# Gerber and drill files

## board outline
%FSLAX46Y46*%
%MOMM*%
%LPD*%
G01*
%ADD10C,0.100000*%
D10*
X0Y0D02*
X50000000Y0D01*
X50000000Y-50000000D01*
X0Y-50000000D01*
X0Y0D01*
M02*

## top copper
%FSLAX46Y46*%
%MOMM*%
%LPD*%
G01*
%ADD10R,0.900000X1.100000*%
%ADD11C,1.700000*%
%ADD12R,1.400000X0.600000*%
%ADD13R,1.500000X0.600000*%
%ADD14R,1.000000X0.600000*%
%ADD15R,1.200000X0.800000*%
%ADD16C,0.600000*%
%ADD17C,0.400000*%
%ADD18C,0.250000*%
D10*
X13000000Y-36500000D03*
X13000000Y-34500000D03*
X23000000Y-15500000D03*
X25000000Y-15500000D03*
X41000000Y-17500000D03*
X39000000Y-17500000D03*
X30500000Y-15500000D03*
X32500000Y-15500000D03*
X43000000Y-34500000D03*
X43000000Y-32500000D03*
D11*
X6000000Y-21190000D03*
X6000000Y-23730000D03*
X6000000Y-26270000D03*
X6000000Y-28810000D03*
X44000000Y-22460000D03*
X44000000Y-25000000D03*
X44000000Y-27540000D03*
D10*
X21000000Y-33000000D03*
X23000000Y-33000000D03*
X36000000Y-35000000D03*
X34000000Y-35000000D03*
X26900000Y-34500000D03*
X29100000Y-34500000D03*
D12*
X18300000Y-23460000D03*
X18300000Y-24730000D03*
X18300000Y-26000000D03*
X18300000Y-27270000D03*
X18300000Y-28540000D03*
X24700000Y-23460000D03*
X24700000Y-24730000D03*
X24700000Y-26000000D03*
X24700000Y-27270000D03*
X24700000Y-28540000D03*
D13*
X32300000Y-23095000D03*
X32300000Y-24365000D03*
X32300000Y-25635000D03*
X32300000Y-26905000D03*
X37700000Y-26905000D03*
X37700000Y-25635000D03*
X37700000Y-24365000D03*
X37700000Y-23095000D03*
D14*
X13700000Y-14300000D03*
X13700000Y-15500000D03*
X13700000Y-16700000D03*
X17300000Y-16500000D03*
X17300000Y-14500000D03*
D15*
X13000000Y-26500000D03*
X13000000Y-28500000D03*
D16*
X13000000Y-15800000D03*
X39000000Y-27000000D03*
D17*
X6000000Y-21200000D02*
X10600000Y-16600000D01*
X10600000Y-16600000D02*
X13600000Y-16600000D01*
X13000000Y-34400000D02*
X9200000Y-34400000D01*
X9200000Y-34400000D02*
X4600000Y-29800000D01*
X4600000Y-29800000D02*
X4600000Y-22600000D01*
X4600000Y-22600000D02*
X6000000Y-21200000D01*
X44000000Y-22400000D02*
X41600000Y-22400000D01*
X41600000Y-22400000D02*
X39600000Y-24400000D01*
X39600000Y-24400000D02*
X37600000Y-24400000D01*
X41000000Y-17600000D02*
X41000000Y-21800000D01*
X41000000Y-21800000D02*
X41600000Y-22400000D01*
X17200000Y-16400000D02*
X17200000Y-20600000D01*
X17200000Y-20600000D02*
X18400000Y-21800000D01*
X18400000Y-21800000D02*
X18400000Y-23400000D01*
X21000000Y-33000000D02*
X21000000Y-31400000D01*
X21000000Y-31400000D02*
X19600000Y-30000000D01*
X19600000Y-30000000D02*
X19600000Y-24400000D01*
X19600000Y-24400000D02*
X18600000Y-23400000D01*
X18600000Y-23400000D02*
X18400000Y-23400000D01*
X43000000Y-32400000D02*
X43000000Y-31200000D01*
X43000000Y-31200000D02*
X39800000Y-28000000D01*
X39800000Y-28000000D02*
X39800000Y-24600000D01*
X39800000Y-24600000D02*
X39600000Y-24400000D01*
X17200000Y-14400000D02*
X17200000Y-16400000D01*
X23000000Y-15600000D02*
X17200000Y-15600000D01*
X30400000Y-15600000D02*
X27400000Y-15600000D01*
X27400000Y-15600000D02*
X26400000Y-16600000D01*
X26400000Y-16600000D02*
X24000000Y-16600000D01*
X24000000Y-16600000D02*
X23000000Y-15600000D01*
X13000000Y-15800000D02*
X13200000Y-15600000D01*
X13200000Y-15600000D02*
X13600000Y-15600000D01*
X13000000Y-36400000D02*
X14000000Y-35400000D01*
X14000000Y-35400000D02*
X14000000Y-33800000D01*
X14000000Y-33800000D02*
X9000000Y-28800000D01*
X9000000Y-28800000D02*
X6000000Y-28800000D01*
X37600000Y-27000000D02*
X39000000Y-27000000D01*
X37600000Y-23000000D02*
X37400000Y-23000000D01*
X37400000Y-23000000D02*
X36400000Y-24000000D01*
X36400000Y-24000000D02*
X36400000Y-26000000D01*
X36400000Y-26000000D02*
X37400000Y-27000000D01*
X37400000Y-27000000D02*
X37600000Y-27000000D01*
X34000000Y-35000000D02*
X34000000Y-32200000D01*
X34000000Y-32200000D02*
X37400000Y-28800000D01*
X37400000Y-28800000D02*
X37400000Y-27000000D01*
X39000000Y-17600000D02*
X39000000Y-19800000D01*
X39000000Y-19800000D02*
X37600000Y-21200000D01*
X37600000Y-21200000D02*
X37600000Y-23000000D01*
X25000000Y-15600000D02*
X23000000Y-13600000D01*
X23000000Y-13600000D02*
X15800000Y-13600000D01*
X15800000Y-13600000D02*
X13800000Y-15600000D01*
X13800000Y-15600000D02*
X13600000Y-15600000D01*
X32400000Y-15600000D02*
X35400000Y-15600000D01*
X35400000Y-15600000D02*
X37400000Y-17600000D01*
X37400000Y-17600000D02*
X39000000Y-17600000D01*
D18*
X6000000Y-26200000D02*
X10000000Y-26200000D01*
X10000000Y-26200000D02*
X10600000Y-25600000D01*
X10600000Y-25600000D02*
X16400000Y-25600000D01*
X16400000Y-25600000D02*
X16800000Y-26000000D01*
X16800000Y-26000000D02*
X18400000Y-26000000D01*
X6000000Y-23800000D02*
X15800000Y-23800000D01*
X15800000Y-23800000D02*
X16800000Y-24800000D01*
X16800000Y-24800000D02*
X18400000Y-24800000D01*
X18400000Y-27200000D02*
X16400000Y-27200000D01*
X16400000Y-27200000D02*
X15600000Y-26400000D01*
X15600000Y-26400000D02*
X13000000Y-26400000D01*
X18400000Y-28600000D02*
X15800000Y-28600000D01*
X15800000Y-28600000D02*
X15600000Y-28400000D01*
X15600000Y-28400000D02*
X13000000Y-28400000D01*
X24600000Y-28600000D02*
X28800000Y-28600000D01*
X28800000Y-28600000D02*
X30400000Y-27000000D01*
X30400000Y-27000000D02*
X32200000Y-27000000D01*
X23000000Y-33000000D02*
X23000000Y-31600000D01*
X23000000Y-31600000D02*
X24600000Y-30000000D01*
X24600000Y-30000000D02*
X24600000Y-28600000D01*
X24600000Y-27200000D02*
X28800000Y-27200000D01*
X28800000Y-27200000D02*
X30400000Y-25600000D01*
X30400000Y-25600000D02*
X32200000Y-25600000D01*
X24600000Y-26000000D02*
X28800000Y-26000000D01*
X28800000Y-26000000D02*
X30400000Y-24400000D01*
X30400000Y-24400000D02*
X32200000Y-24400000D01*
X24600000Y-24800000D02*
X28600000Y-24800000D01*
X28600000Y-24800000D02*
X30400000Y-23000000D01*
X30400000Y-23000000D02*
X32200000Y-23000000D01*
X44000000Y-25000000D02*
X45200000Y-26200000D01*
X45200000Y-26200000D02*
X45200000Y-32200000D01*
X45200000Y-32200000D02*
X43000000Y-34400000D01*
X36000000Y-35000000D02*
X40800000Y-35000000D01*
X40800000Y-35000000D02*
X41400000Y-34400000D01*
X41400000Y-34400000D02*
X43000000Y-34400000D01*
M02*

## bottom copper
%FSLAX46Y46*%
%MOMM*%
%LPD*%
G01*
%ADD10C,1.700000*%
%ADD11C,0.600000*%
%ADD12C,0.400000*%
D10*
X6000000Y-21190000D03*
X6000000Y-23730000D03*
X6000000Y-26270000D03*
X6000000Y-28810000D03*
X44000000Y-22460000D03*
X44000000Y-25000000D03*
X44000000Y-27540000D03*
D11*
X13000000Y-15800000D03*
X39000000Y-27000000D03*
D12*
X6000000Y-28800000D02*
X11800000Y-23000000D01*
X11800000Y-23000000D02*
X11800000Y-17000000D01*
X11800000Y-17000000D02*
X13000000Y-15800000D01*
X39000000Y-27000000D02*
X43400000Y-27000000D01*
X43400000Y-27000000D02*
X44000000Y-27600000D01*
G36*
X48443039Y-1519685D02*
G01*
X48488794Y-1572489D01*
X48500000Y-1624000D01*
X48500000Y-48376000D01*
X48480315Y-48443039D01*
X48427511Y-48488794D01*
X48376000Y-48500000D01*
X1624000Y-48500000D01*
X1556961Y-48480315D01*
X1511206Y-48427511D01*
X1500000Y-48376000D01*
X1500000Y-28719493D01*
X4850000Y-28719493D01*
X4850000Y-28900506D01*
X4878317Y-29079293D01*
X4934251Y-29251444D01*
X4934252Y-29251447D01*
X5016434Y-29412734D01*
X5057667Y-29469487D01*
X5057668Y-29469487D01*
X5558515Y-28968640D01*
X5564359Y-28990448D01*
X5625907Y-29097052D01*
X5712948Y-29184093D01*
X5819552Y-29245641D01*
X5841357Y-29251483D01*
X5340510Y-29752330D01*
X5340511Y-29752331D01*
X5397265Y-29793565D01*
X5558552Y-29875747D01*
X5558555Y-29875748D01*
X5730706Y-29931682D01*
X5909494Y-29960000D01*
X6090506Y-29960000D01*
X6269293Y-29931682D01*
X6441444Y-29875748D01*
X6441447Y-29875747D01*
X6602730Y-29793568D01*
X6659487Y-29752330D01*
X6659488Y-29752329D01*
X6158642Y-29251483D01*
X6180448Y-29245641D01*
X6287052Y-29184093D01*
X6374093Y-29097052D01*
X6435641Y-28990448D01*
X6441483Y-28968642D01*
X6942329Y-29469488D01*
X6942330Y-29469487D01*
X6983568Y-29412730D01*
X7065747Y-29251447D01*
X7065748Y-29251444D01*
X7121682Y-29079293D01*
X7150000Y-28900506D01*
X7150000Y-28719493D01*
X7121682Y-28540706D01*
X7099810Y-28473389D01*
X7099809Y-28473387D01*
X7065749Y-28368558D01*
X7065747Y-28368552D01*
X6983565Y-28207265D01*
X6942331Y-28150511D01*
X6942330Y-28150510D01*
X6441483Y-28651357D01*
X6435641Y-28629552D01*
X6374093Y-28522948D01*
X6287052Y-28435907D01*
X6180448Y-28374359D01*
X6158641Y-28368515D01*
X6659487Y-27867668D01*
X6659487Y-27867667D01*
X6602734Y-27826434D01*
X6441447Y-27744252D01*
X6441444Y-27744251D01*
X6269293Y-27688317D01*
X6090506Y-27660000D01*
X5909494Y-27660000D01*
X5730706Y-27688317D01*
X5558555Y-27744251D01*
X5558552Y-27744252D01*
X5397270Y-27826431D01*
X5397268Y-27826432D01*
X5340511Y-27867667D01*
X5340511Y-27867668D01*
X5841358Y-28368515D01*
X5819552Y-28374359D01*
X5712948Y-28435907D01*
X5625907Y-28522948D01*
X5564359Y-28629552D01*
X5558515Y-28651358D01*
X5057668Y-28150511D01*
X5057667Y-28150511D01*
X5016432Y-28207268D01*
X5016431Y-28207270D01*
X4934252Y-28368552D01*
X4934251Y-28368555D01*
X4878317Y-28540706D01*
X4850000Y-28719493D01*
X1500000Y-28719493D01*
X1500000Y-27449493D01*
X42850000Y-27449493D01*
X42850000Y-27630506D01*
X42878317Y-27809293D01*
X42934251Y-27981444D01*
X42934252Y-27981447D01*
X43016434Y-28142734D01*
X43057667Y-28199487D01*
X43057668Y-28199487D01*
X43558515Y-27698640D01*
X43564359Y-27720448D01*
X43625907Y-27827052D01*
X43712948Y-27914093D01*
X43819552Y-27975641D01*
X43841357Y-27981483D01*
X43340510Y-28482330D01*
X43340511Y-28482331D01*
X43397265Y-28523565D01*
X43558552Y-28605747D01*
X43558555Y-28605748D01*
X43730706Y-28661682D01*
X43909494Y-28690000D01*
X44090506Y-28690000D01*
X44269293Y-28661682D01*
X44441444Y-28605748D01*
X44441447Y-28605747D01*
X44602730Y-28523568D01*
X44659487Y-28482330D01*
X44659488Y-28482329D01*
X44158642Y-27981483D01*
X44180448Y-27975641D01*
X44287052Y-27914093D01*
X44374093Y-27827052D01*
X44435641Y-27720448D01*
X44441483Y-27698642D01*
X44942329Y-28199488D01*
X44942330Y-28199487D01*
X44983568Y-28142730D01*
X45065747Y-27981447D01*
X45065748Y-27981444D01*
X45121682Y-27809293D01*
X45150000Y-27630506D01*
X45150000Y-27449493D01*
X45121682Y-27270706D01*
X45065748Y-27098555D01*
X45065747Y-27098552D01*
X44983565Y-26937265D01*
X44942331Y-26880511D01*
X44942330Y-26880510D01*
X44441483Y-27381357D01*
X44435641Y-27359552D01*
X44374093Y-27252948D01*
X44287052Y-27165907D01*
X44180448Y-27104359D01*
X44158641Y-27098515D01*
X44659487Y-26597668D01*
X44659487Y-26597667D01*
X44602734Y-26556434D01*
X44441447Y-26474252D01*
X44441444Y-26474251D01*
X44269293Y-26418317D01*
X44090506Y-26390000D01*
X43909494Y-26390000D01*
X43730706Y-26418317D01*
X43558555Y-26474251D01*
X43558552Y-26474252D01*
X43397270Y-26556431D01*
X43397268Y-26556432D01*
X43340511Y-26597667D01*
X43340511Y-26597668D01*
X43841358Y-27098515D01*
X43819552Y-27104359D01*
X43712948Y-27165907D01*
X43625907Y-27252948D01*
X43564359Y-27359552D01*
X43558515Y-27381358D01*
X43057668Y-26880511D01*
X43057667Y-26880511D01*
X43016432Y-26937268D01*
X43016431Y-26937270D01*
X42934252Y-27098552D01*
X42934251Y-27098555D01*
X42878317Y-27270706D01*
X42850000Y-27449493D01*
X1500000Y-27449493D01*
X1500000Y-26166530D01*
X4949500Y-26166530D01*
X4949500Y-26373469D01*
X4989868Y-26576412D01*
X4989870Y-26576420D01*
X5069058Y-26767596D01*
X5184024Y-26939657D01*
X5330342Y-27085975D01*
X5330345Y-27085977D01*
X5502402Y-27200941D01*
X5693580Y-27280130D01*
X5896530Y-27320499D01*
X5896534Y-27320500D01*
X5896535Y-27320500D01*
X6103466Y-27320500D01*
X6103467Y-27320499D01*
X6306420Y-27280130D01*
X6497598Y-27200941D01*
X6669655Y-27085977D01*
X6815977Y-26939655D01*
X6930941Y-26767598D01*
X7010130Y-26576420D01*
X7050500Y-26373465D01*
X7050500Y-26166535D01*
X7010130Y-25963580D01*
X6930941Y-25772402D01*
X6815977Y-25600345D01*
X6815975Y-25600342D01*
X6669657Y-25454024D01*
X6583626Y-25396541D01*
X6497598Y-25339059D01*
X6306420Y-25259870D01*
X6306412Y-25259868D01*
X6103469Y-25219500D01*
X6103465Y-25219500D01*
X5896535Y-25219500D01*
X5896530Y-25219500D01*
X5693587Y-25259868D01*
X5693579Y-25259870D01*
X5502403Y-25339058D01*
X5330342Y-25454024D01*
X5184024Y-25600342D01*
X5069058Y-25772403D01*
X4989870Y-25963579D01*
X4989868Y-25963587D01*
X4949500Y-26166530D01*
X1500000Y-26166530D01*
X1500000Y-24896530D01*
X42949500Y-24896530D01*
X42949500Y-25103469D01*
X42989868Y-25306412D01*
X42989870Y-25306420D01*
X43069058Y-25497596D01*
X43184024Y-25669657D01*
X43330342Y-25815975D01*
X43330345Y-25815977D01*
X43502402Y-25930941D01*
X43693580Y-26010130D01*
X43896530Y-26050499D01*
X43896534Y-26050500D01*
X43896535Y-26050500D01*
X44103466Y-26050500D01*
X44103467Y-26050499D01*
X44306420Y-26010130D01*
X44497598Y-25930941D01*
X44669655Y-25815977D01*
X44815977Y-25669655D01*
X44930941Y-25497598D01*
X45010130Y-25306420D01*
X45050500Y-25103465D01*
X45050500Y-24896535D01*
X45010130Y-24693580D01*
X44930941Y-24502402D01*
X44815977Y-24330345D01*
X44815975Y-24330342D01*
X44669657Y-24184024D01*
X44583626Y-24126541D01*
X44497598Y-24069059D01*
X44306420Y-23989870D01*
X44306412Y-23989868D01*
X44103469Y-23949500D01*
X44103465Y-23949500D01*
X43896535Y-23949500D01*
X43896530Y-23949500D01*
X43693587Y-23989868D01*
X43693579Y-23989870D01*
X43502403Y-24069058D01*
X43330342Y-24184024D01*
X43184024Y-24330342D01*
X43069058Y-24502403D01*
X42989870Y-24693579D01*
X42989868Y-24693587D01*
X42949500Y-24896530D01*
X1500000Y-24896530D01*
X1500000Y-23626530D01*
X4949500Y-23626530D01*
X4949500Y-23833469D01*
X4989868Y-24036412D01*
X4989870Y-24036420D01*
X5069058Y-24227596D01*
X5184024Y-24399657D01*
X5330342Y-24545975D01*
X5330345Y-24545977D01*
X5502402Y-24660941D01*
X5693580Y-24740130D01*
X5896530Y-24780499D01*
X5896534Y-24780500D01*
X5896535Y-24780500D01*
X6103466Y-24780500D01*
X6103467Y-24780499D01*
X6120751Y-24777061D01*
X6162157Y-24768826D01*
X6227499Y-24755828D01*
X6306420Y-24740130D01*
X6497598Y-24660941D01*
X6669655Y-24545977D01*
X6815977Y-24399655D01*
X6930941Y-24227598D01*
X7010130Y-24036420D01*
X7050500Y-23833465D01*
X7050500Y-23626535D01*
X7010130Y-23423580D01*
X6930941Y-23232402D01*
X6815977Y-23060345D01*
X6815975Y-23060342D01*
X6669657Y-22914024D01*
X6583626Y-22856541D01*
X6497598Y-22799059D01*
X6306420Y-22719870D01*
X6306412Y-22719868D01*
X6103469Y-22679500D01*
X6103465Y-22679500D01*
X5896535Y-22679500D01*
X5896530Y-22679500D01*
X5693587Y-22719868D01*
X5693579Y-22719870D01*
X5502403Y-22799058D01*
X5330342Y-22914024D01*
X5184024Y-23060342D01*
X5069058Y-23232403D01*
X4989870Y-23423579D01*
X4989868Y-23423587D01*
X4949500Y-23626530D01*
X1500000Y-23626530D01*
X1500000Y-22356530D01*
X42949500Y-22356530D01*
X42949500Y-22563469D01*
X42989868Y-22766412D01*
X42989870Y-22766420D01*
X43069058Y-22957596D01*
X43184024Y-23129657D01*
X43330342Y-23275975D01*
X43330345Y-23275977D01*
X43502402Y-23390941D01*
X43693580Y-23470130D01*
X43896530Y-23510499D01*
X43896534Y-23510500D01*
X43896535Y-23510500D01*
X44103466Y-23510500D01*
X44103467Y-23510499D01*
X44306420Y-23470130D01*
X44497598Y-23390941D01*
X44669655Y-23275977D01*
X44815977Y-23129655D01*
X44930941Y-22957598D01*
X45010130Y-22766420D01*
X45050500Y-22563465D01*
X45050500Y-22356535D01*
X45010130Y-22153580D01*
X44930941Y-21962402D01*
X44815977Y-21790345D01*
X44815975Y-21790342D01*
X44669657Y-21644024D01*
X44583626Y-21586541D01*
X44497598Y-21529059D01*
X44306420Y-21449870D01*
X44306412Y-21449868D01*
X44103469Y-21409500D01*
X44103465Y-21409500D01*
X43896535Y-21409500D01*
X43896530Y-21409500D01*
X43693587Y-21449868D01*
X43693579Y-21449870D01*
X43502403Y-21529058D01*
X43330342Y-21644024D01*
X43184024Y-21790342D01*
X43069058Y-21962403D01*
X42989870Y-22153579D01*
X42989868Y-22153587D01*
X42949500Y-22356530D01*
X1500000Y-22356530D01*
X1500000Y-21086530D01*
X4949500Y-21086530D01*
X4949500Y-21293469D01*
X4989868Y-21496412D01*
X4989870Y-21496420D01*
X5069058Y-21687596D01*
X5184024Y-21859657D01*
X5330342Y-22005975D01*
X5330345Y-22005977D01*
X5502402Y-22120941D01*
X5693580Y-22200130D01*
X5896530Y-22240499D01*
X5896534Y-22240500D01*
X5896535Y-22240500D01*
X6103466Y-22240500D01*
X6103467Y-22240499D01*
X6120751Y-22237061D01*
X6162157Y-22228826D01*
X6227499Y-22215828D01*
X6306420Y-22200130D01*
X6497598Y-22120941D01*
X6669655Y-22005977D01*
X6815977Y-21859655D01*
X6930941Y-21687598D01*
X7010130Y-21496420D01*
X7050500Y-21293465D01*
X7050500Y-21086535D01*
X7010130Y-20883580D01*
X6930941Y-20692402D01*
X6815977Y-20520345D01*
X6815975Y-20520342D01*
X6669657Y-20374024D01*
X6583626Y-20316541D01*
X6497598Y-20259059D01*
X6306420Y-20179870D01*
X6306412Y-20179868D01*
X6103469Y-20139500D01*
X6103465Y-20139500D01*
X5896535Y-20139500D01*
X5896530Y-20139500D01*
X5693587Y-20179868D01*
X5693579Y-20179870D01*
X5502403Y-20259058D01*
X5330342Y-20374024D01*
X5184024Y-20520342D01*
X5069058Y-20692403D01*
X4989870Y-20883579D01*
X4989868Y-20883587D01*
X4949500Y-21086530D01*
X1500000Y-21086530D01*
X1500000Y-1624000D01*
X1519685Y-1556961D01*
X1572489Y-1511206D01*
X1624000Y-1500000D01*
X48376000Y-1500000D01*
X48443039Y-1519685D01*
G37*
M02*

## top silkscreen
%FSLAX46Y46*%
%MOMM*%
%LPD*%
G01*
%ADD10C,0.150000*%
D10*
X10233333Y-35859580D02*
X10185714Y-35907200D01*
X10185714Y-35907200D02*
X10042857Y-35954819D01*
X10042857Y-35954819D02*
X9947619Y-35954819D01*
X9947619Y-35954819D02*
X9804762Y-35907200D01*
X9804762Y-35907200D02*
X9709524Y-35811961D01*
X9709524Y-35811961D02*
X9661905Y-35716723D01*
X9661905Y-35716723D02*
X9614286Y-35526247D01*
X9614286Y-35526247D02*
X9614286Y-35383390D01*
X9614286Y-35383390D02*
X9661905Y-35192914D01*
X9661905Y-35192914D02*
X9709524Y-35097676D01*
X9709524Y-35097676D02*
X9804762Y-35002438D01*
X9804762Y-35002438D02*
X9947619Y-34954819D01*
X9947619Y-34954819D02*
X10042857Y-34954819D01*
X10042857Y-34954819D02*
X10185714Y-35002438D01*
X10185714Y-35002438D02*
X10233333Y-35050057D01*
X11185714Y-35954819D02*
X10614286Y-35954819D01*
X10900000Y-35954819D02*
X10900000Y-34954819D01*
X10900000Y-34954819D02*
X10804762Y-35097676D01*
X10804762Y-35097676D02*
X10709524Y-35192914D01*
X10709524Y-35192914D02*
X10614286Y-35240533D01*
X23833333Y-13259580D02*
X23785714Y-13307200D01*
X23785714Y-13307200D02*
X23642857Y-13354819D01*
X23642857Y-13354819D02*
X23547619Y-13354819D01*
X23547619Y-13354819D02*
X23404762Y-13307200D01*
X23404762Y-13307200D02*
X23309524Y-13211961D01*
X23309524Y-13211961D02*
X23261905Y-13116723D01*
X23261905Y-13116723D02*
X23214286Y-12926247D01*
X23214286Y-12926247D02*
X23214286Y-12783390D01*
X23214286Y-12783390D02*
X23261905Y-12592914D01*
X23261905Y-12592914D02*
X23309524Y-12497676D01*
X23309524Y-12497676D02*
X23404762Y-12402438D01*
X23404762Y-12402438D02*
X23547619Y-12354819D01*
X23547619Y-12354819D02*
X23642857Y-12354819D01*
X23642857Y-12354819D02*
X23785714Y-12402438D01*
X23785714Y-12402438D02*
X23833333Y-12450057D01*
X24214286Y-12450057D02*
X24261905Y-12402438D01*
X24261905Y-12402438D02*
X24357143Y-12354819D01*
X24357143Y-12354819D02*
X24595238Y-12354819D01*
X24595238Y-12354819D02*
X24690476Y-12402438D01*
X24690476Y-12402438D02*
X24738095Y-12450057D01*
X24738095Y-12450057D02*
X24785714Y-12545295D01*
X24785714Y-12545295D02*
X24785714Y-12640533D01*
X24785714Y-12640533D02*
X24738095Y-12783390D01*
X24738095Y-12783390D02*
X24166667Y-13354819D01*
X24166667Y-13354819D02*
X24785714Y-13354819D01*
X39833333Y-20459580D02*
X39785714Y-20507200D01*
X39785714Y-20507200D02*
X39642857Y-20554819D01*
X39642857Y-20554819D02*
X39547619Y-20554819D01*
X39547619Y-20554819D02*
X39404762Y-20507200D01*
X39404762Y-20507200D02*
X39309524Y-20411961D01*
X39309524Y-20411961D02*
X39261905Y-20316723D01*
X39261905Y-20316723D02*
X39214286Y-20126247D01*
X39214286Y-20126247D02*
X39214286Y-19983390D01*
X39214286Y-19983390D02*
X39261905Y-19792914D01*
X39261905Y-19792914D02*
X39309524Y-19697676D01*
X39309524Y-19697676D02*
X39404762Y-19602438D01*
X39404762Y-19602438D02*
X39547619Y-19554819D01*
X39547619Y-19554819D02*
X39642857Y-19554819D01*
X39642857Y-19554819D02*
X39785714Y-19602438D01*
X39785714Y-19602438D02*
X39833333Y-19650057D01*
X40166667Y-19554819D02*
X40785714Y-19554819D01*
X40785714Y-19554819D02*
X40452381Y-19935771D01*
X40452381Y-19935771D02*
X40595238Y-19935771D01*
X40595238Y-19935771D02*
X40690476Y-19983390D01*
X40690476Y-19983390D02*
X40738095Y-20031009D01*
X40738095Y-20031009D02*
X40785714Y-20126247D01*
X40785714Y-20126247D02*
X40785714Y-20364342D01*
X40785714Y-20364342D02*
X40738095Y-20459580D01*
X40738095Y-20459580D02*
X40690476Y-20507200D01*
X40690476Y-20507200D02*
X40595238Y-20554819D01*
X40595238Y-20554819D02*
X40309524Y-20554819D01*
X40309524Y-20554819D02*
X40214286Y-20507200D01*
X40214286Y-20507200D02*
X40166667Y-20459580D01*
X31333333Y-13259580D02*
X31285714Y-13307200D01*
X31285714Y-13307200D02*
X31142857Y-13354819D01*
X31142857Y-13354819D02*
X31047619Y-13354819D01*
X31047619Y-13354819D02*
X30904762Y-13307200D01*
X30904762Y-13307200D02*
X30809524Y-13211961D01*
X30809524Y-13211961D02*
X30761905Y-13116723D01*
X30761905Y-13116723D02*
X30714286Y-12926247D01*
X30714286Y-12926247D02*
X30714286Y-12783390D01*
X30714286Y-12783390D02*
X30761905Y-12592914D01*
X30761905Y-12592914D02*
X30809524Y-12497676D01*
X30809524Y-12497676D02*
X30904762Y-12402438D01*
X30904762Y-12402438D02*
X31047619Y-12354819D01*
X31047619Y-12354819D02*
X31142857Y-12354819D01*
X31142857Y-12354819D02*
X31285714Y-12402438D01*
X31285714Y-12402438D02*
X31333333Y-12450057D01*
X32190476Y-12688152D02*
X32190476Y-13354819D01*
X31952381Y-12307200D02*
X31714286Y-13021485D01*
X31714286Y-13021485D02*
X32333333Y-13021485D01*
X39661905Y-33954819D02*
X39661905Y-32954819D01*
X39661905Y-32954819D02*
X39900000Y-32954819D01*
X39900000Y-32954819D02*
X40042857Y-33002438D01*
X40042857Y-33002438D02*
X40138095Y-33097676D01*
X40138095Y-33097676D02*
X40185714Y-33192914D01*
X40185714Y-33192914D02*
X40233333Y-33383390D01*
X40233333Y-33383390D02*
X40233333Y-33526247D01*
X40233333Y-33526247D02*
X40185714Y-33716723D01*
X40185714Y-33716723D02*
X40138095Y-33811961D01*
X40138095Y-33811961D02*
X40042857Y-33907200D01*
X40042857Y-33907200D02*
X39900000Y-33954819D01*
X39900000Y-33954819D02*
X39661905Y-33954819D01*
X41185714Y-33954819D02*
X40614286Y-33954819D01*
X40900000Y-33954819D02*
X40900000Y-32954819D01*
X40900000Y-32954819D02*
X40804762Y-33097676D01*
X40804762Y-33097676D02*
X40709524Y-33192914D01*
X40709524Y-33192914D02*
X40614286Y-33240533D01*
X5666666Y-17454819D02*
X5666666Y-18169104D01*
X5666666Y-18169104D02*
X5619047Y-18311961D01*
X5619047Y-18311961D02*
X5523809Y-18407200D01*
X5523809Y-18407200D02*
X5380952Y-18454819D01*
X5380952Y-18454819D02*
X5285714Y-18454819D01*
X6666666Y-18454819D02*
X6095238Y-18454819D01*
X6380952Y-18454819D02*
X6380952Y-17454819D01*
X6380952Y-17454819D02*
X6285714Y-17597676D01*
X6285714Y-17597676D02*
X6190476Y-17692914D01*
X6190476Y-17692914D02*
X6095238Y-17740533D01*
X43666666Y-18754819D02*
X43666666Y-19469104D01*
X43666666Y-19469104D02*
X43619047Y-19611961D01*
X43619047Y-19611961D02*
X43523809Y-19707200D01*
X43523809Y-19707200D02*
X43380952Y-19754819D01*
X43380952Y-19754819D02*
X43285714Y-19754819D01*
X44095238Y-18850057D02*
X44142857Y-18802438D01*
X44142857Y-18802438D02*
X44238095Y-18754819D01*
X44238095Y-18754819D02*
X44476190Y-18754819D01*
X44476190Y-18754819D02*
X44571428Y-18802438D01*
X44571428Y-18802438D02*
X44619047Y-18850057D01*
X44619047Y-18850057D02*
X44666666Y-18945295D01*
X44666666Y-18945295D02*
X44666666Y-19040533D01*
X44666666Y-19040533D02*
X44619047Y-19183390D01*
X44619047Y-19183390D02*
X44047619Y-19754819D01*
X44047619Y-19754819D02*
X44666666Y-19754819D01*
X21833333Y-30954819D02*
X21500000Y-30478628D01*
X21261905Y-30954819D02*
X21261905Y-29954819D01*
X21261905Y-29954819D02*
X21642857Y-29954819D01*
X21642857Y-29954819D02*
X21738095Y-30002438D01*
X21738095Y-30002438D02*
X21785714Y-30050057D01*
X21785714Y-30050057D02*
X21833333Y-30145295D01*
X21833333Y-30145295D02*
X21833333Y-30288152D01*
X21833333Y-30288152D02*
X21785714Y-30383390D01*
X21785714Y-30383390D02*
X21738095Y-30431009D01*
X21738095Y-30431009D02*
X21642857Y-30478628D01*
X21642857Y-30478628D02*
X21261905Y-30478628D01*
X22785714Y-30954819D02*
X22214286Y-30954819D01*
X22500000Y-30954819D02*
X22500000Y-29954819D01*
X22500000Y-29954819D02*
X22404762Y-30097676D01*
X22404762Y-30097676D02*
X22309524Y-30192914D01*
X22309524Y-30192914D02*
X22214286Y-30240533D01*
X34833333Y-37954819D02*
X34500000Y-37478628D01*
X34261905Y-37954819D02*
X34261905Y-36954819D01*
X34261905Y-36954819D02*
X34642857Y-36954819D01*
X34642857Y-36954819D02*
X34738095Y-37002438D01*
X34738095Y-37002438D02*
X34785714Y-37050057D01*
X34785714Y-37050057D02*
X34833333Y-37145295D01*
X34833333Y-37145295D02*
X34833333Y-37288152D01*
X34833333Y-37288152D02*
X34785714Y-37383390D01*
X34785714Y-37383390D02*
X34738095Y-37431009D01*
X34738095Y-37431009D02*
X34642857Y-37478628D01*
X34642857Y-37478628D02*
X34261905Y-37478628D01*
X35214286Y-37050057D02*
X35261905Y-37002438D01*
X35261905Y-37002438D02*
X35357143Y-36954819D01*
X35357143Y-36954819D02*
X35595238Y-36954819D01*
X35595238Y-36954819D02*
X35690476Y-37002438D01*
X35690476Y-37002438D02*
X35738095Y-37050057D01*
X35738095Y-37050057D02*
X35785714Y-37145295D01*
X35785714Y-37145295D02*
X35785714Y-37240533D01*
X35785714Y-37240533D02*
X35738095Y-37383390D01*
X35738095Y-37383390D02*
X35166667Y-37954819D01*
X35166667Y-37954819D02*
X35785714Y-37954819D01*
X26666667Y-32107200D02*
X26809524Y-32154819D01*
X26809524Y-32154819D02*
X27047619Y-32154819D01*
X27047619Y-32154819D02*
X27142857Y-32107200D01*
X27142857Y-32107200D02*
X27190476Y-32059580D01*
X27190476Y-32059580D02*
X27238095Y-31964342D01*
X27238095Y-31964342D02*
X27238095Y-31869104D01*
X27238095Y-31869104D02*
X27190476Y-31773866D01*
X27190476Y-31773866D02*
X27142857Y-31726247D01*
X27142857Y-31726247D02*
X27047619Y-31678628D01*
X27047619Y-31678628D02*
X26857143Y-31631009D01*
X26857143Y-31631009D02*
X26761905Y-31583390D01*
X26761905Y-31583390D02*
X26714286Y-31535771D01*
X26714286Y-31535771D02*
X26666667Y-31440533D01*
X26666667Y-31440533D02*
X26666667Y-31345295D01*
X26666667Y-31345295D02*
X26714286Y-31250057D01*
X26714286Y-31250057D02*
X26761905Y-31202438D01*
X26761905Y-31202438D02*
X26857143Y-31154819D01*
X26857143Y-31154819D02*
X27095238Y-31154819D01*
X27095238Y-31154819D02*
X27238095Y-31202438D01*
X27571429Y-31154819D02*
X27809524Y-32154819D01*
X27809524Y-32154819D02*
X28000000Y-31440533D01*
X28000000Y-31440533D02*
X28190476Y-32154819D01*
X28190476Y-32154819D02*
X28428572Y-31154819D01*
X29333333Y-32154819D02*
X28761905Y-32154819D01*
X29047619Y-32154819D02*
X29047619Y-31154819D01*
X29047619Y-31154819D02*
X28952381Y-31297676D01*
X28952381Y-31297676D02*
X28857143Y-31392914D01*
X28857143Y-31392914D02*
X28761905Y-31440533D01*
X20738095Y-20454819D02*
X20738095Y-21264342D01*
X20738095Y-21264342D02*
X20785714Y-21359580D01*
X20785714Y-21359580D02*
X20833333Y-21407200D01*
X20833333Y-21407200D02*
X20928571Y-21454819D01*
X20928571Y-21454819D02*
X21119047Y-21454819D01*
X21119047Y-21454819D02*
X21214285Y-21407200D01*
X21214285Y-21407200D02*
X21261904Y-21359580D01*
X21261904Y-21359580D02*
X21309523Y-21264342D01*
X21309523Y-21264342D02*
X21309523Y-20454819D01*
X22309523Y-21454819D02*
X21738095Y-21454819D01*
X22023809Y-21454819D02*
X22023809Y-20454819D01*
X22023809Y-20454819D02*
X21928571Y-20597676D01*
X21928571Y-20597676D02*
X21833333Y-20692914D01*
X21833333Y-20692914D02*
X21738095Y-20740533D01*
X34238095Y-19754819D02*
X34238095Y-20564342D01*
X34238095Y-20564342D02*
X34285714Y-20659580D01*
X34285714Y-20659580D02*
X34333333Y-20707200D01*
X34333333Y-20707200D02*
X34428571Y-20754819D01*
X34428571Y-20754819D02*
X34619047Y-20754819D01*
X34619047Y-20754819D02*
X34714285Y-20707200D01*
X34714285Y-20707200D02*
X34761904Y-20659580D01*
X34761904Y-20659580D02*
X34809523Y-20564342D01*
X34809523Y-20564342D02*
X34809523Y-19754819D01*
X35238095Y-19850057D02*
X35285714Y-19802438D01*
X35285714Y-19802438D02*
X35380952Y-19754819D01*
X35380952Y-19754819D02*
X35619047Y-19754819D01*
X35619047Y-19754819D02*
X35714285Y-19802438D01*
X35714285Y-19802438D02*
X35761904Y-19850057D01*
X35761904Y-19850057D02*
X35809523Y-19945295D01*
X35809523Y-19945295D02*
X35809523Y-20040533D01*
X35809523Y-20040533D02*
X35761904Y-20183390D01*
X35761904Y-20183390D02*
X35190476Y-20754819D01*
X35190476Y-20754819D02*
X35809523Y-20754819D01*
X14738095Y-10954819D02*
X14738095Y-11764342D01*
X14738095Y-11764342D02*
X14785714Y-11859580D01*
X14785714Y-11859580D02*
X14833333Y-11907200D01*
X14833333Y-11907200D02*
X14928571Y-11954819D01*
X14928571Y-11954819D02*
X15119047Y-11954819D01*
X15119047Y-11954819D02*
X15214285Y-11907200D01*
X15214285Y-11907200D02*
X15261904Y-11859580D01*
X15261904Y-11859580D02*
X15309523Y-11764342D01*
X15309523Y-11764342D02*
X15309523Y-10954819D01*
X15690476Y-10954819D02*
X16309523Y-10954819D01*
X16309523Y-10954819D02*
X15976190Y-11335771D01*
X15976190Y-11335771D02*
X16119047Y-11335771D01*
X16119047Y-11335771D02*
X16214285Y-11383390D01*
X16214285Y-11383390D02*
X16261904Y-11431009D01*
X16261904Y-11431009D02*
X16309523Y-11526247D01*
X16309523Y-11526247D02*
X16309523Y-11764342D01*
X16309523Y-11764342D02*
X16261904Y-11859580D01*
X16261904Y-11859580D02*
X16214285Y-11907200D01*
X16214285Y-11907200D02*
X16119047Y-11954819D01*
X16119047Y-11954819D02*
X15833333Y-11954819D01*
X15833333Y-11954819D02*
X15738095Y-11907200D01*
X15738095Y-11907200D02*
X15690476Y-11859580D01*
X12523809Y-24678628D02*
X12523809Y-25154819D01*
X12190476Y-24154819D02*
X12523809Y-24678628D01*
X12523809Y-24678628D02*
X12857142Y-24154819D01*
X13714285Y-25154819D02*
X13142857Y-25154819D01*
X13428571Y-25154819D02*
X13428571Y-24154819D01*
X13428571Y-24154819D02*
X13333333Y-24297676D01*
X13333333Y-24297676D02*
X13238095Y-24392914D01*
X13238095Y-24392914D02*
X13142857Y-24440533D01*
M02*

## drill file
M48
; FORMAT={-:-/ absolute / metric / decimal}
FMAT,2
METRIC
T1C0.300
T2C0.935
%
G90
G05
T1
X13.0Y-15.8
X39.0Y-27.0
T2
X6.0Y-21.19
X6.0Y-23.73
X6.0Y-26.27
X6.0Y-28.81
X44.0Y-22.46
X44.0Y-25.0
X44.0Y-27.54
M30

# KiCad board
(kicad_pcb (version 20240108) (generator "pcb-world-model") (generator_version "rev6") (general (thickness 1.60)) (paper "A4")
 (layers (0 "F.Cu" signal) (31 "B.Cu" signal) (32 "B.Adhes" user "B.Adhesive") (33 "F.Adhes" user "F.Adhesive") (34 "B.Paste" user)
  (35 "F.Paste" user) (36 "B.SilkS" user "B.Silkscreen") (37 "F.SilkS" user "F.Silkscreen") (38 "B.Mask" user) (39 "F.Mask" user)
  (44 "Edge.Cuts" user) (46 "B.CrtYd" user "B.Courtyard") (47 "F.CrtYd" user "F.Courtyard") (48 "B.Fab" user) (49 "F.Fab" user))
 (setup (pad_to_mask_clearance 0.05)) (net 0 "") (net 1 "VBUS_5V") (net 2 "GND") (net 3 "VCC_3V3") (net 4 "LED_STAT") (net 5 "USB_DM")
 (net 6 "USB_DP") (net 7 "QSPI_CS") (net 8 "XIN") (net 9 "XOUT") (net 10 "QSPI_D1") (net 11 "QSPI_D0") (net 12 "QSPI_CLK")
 (gr_rect (start 0.0 0.0) (end 50.0000 50.0000) (stroke (width 0.1) (type default)) (fill none) (layer "Edge.Cuts"))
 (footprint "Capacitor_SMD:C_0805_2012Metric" (layer "F.Cu") (at 13.0000 35.5000 90)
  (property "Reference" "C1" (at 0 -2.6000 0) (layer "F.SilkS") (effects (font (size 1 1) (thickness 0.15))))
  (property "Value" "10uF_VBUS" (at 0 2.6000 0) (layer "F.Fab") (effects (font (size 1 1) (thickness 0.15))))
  (pad "1" smd rect (at -1.0000 0.0000) (size 0.9000 1.1000) (layers "F.Cu" "F.Paste" "F.Mask") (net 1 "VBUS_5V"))
  (pad "2" smd rect (at 1.0000 0.0000) (size 0.9000 1.1000) (layers "F.Cu" "F.Paste" "F.Mask") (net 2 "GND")))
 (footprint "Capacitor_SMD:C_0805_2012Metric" (layer "F.Cu") (at 24.0000 15.5000 0)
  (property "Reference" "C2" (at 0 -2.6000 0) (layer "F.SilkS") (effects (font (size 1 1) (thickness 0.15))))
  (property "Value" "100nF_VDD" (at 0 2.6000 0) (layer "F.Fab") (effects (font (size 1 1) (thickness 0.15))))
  (pad "1" smd rect (at -1.0000 0.0000) (size 0.9000 1.1000) (layers "F.Cu" "F.Paste" "F.Mask") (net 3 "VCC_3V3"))
  (pad "2" smd rect (at 1.0000 0.0000) (size 0.9000 1.1000) (layers "F.Cu" "F.Paste" "F.Mask") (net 2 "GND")))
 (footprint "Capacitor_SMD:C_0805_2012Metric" (layer "F.Cu") (at 40.0000 17.5000 180)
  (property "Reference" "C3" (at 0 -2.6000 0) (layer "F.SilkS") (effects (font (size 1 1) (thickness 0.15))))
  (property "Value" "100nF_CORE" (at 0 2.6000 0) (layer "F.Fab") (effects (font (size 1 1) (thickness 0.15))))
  (pad "1" smd rect (at -1.0000 0.0000) (size 0.9000 1.1000) (layers "F.Cu" "F.Paste" "F.Mask") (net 3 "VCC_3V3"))
  (pad "2" smd rect (at 1.0000 0.0000) (size 0.9000 1.1000) (layers "F.Cu" "F.Paste" "F.Mask") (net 2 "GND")))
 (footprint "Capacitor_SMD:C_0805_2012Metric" (layer "F.Cu") (at 31.5000 15.5000 0)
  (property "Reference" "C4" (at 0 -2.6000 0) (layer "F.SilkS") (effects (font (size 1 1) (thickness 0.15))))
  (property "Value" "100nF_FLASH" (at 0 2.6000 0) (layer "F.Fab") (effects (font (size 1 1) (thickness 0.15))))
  (pad "1" smd rect (at -1.0000 0.0000) (size 0.9000 1.1000) (layers "F.Cu" "F.Paste" "F.Mask") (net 3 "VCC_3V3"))
  (pad "2" smd rect (at 1.0000 0.0000) (size 0.9000 1.1000) (layers "F.Cu" "F.Paste" "F.Mask") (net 2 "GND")))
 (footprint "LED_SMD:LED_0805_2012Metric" (layer "F.Cu") (at 43.0000 33.5000 90)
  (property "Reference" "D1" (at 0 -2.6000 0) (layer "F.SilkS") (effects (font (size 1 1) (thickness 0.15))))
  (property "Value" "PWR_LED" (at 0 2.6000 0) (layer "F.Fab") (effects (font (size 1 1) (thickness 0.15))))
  (pad "1" smd rect (at -1.0000 0.0000) (size 0.9000 1.1000) (layers "F.Cu" "F.Paste" "F.Mask") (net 3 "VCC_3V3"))
  (pad "2" smd rect (at 1.0000 0.0000) (size 0.9000 1.1000) (layers "F.Cu" "F.Paste" "F.Mask") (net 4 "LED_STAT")))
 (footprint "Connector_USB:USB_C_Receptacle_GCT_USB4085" (layer "F.Cu") (at 6.0000 25.0000 0) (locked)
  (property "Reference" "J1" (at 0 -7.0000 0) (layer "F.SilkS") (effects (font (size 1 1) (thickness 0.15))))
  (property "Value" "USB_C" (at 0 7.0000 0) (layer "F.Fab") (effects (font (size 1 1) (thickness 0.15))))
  (pad "1" thru_hole circle (at 0.0000 -3.8100) (size 1.7000 1.7000) (drill 0.9350) (layers "*.Cu" "*.Mask") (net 1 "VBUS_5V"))
  (pad "2" thru_hole circle (at 0.0000 -1.2700) (size 1.7000 1.7000) (drill 0.9350) (layers "*.Cu" "*.Mask") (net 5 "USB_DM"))
  (pad "3" thru_hole circle (at 0.0000 1.2700) (size 1.7000 1.7000) (drill 0.9350) (layers "*.Cu" "*.Mask") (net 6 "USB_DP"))
  (pad "4" thru_hole circle (at 0.0000 3.8100) (size 1.7000 1.7000) (drill 0.9350) (layers "*.Cu" "*.Mask") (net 2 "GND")))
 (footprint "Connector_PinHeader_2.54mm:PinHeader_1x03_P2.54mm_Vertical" (layer "F.Cu") (at 44.0000 25.0000 0) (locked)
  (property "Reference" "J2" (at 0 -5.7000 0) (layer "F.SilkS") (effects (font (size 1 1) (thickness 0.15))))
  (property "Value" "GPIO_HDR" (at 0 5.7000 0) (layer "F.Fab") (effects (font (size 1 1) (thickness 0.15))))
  (pad "1" thru_hole circle (at 0.0000 -2.5400) (size 1.7000 1.7000) (drill 0.9350) (layers "*.Cu" "*.Mask") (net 3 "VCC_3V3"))
  (pad "2" thru_hole circle (at 0.0000 0.0000) (size 1.7000 1.7000) (drill 0.9350) (layers "*.Cu" "*.Mask") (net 4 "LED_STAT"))
  (pad "3" thru_hole circle (at 0.0000 2.5400) (size 1.7000 1.7000) (drill 0.9350) (layers "*.Cu" "*.Mask") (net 2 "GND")))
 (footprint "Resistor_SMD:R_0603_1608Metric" (layer "F.Cu") (at 22.0000 33.0000 0)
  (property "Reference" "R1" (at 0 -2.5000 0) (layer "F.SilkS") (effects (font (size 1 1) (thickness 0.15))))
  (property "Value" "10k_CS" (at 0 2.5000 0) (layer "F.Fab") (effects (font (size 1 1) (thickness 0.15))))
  (pad "1" smd rect (at -1.0000 0.0000) (size 0.9000 1.1000) (layers "F.Cu" "F.Paste" "F.Mask") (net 3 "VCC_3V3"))
  (pad "2" smd rect (at 1.0000 0.0000) (size 0.9000 1.1000) (layers "F.Cu" "F.Paste" "F.Mask") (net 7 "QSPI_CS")))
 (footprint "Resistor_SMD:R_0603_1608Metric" (layer "F.Cu") (at 35.0000 35.0000 180)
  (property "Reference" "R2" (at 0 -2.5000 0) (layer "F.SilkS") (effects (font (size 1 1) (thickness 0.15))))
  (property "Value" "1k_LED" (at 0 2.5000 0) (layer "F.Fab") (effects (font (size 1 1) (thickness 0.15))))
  (pad "1" smd rect (at -1.0000 0.0000) (size 0.9000 1.1000) (layers "F.Cu" "F.Paste" "F.Mask") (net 4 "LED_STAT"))
  (pad "2" smd rect (at 1.0000 0.0000) (size 0.9000 1.1000) (layers "F.Cu" "F.Paste" "F.Mask") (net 2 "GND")))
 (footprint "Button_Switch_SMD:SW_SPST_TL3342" (layer "F.Cu") (at 28.0000 34.5000 0)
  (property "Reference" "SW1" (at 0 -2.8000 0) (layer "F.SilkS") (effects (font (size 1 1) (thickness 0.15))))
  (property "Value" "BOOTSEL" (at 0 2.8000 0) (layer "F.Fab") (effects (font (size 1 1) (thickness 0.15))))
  (pad "1" smd rect (at -1.1000 0.0000) (size 0.9000 1.1000) (layers "F.Cu" "F.Paste" "F.Mask") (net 7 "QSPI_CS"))
  (pad "2" smd rect (at 1.1000 0.0000) (size 0.9000 1.1000) (layers "F.Cu" "F.Paste" "F.Mask") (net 2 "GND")))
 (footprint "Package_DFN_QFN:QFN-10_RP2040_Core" (layer "F.Cu") (at 21.5000 26.0000 0)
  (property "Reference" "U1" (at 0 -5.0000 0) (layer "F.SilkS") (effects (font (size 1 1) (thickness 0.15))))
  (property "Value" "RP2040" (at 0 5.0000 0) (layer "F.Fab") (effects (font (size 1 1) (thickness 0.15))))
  (pad "1" smd rect (at -3.2000 -2.5400) (size 1.4000 0.6000) (layers "F.Cu" "F.Paste" "F.Mask") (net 3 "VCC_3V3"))
  (pad "2" smd rect (at -3.2000 -1.2700) (size 1.4000 0.6000) (layers "F.Cu" "F.Paste" "F.Mask") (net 5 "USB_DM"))
  (pad "3" smd rect (at -3.2000 0.0000) (size 1.4000 0.6000) (layers "F.Cu" "F.Paste" "F.Mask") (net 6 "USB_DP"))
  (pad "4" smd rect (at -3.2000 1.2700) (size 1.4000 0.6000) (layers "F.Cu" "F.Paste" "F.Mask") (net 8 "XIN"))
  (pad "5" smd rect (at -3.2000 2.5400) (size 1.4000 0.6000) (layers "F.Cu" "F.Paste" "F.Mask") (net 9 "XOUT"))
  (pad "6" smd rect (at 3.2000 -2.5400) (size 1.4000 0.6000) (layers "F.Cu" "F.Paste" "F.Mask") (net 4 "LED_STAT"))
  (pad "7" smd rect (at 3.2000 -1.2700) (size 1.4000 0.6000) (layers "F.Cu" "F.Paste" "F.Mask") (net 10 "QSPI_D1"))
  (pad "8" smd rect (at 3.2000 0.0000) (size 1.4000 0.6000) (layers "F.Cu" "F.Paste" "F.Mask") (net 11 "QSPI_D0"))
  (pad "9" smd rect (at 3.2000 1.2700) (size 1.4000 0.6000) (layers "F.Cu" "F.Paste" "F.Mask") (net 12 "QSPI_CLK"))
  (pad "10" smd rect (at 3.2000 2.5400) (size 1.4000 0.6000) (layers "F.Cu" "F.Paste" "F.Mask") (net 7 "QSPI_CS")))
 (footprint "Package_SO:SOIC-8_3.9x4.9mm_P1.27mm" (layer "F.Cu") (at 35.0000 25.0000 0)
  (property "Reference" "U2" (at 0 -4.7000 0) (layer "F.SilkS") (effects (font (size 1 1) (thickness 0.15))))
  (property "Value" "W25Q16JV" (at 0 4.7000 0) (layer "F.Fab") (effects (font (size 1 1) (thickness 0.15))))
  (pad "1" smd rect (at -2.7000 -1.9050) (size 1.5000 0.6000) (layers "F.Cu" "F.Paste" "F.Mask") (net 10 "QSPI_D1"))
  (pad "2" smd rect (at -2.7000 -0.6350) (size 1.5000 0.6000) (layers "F.Cu" "F.Paste" "F.Mask") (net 11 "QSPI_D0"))
  (pad "3" smd rect (at -2.7000 0.6350) (size 1.5000 0.6000) (layers "F.Cu" "F.Paste" "F.Mask") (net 12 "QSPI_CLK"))
  (pad "4" smd rect (at -2.7000 1.9050) (size 1.5000 0.6000) (layers "F.Cu" "F.Paste" "F.Mask") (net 7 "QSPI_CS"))
  (pad "5" smd rect (at 2.7000 1.9050) (size 1.5000 0.6000) (layers "F.Cu" "F.Paste" "F.Mask") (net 2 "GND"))
  (pad "6" smd rect (at 2.7000 0.6350) (size 1.5000 0.6000) (layers "F.Cu" "F.Paste" "F.Mask") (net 3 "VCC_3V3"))
  (pad "7" smd rect (at 2.7000 -0.6350) (size 1.5000 0.6000) (layers "F.Cu" "F.Paste" "F.Mask") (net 3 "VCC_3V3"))
  (pad "8" smd rect (at 2.7000 -1.9050) (size 1.5000 0.6000) (layers "F.Cu" "F.Paste" "F.Mask") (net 2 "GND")))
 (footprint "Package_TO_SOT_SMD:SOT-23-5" (layer "F.Cu") (at 15.5000 15.5000 0)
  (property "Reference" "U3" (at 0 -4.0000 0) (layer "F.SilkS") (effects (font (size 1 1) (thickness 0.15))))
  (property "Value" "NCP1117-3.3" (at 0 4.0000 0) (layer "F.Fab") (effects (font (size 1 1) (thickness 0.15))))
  (pad "1" smd rect (at -1.8000 -1.2000) (size 1.0000 0.6000) (layers "F.Cu" "F.Paste" "F.Mask") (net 1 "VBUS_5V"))
  (pad "2" smd rect (at -1.8000 0.0000) (size 1.0000 0.6000) (layers "F.Cu" "F.Paste" "F.Mask") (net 2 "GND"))
  (pad "3" smd rect (at -1.8000 1.2000) (size 1.0000 0.6000) (layers "F.Cu" "F.Paste" "F.Mask") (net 1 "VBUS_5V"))
  (pad "4" smd rect (at 1.8000 1.0000) (size 1.0000 0.6000) (layers "F.Cu" "F.Paste" "F.Mask") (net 3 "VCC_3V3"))
  (pad "5" smd rect (at 1.8000 -1.0000) (size 1.0000 0.6000) (layers "F.Cu" "F.Paste" "F.Mask") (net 3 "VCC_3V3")))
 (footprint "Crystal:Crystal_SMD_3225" (layer "F.Cu") (at 13.0000 27.5000 0)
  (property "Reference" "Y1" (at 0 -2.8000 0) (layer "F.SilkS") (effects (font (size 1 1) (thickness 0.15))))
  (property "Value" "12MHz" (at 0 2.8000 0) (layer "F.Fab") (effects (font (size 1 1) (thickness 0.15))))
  (pad "1" smd rect (at 0.0000 -1.0000) (size 1.2000 0.8000) (layers "F.Cu" "F.Paste" "F.Mask") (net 8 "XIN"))
  (pad "2" smd rect (at 0.0000 1.0000) (size 1.2000 0.8000) (layers "F.Cu" "F.Paste" "F.Mask") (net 9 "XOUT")))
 (segment (start 6.0000 21.2000) (end 10.6000 16.6000) (width 0.4000) (layer "F.Cu") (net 1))
 (segment (start 10.6000 16.6000) (end 13.6000 16.6000) (width 0.4000) (layer "F.Cu") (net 1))
 (segment (start 13.0000 34.4000) (end 9.2000 34.4000) (width 0.4000) (layer "F.Cu") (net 1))
 (segment (start 9.2000 34.4000) (end 4.6000 29.8000) (width 0.4000) (layer "F.Cu") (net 1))
 (segment (start 4.6000 29.8000) (end 4.6000 22.6000) (width 0.4000) (layer "F.Cu") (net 1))
 (segment (start 4.6000 22.6000) (end 6.0000 21.2000) (width 0.4000) (layer "F.Cu") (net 1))
 (segment (start 44.0000 22.4000) (end 41.6000 22.4000) (width 0.4000) (layer "F.Cu") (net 3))
 (segment (start 41.6000 22.4000) (end 39.6000 24.4000) (width 0.4000) (layer "F.Cu") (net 3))
 (segment (start 39.6000 24.4000) (end 37.6000 24.4000) (width 0.4000) (layer "F.Cu") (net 3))
 (segment (start 41.0000 17.6000) (end 41.0000 21.8000) (width 0.4000) (layer "F.Cu") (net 3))
 (segment (start 41.0000 21.8000) (end 41.6000 22.4000) (width 0.4000) (layer "F.Cu") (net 3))
 (segment (start 17.2000 16.4000) (end 17.2000 20.6000) (width 0.4000) (layer "F.Cu") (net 3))
 (segment (start 17.2000 20.6000) (end 18.4000 21.8000) (width 0.4000) (layer "F.Cu") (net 3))
 (segment (start 18.4000 21.8000) (end 18.4000 23.4000) (width 0.4000) (layer "F.Cu") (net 3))
 (segment (start 21.0000 33.0000) (end 21.0000 31.4000) (width 0.4000) (layer "F.Cu") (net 3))
 (segment (start 21.0000 31.4000) (end 19.6000 30.0000) (width 0.4000) (layer "F.Cu") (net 3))
 (segment (start 19.6000 30.0000) (end 19.6000 24.4000) (width 0.4000) (layer "F.Cu") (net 3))
 (segment (start 19.6000 24.4000) (end 18.6000 23.4000) (width 0.4000) (layer "F.Cu") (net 3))
 (segment (start 18.6000 23.4000) (end 18.4000 23.4000) (width 0.4000) (layer "F.Cu") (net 3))
 (segment (start 43.0000 32.4000) (end 43.0000 31.2000) (width 0.4000) (layer "F.Cu") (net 3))
 (segment (start 43.0000 31.2000) (end 39.8000 28.0000) (width 0.4000) (layer "F.Cu") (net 3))
 (segment (start 39.8000 28.0000) (end 39.8000 24.6000) (width 0.4000) (layer "F.Cu") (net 3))
 (segment (start 39.8000 24.6000) (end 39.6000 24.4000) (width 0.4000) (layer "F.Cu") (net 3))
 (segment (start 17.2000 14.4000) (end 17.2000 16.4000) (width 0.4000) (layer "F.Cu") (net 3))
 (segment (start 23.0000 15.6000) (end 17.2000 15.6000) (width 0.4000) (layer "F.Cu") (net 3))
 (segment (start 30.4000 15.6000) (end 27.4000 15.6000) (width 0.4000) (layer "F.Cu") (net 3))
 (segment (start 27.4000 15.6000) (end 26.4000 16.6000) (width 0.4000) (layer "F.Cu") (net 3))
 (segment (start 26.4000 16.6000) (end 24.0000 16.6000) (width 0.4000) (layer "F.Cu") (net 3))
 (segment (start 24.0000 16.6000) (end 23.0000 15.6000) (width 0.4000) (layer "F.Cu") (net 3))
 (segment (start 6.0000 28.8000) (end 11.8000 23.0000) (width 0.4000) (layer "B.Cu") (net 2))
 (segment (start 11.8000 23.0000) (end 11.8000 17.0000) (width 0.4000) (layer "B.Cu") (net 2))
 (segment (start 11.8000 17.0000) (end 13.0000 15.8000) (width 0.4000) (layer "B.Cu") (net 2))
 (segment (start 13.0000 15.8000) (end 13.2000 15.6000) (width 0.4000) (layer "F.Cu") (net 2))
 (segment (start 13.2000 15.6000) (end 13.6000 15.6000) (width 0.4000) (layer "F.Cu") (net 2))
 (segment (start 13.0000 36.4000) (end 14.0000 35.4000) (width 0.4000) (layer "F.Cu") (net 2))
 (segment (start 14.0000 35.4000) (end 14.0000 33.8000) (width 0.4000) (layer "F.Cu") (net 2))
 (segment (start 14.0000 33.8000) (end 9.0000 28.8000) (width 0.4000) (layer "F.Cu") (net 2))
 (segment (start 9.0000 28.8000) (end 6.0000 28.8000) (width 0.4000) (layer "F.Cu") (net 2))
 (segment (start 37.6000 27.0000) (end 39.0000 27.0000) (width 0.4000) (layer "F.Cu") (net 2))
 (segment (start 39.0000 27.0000) (end 43.4000 27.0000) (width 0.4000) (layer "B.Cu") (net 2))
 (segment (start 43.4000 27.0000) (end 44.0000 27.6000) (width 0.4000) (layer "B.Cu") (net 2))
 (segment (start 37.6000 23.0000) (end 37.4000 23.0000) (width 0.4000) (layer "F.Cu") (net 2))
 (segment (start 37.4000 23.0000) (end 36.4000 24.0000) (width 0.4000) (layer "F.Cu") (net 2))
 (segment (start 36.4000 24.0000) (end 36.4000 26.0000) (width 0.4000) (layer "F.Cu") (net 2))
 (segment (start 36.4000 26.0000) (end 37.4000 27.0000) (width 0.4000) (layer "F.Cu") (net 2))
 (segment (start 37.4000 27.0000) (end 37.6000 27.0000) (width 0.4000) (layer "F.Cu") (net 2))
 (segment (start 34.0000 35.0000) (end 34.0000 32.2000) (width 0.4000) (layer "F.Cu") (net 2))
 (segment (start 34.0000 32.2000) (end 37.4000 28.8000) (width 0.4000) (layer "F.Cu") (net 2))
 (segment (start 37.4000 28.8000) (end 37.4000 27.0000) (width 0.4000) (layer "F.Cu") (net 2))
 (segment (start 39.0000 17.6000) (end 39.0000 19.8000) (width 0.4000) (layer "F.Cu") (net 2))
 (segment (start 39.0000 19.8000) (end 37.6000 21.2000) (width 0.4000) (layer "F.Cu") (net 2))
 (segment (start 37.6000 21.2000) (end 37.6000 23.0000) (width 0.4000) (layer "F.Cu") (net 2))
 (segment (start 25.0000 15.6000) (end 23.0000 13.6000) (width 0.4000) (layer "F.Cu") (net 2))
 (segment (start 23.0000 13.6000) (end 15.8000 13.6000) (width 0.4000) (layer "F.Cu") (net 2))
 (segment (start 15.8000 13.6000) (end 13.8000 15.6000) (width 0.4000) (layer "F.Cu") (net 2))
 (segment (start 13.8000 15.6000) (end 13.6000 15.6000) (width 0.4000) (layer "F.Cu") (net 2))
 (segment (start 32.4000 15.6000) (end 35.4000 15.6000) (width 0.4000) (layer "F.Cu") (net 2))
 (segment (start 35.4000 15.6000) (end 37.4000 17.6000) (width 0.4000) (layer "F.Cu") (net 2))
 (segment (start 37.4000 17.6000) (end 39.0000 17.6000) (width 0.4000) (layer "F.Cu") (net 2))
 (segment (start 6.0000 26.2000) (end 10.0000 26.2000) (width 0.2500) (layer "F.Cu") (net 6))
 (segment (start 10.0000 26.2000) (end 10.6000 25.6000) (width 0.2500) (layer "F.Cu") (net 6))
 (segment (start 10.6000 25.6000) (end 16.4000 25.6000) (width 0.2500) (layer "F.Cu") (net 6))
 (segment (start 16.4000 25.6000) (end 16.8000 26.0000) (width 0.2500) (layer "F.Cu") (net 6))
 (segment (start 16.8000 26.0000) (end 18.4000 26.0000) (width 0.2500) (layer "F.Cu") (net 6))
 (segment (start 6.0000 23.8000) (end 15.8000 23.8000) (width 0.2500) (layer "F.Cu") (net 5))
 (segment (start 15.8000 23.8000) (end 16.8000 24.8000) (width 0.2500) (layer "F.Cu") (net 5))
 (segment (start 16.8000 24.8000) (end 18.4000 24.8000) (width 0.2500) (layer "F.Cu") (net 5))
 (segment (start 18.4000 27.2000) (end 16.4000 27.2000) (width 0.2500) (layer "F.Cu") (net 8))
 (segment (start 16.4000 27.2000) (end 15.6000 26.4000) (width 0.2500) (layer "F.Cu") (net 8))
 (segment (start 15.6000 26.4000) (end 13.0000 26.4000) (width 0.2500) (layer "F.Cu") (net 8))
 (segment (start 18.4000 28.6000) (end 15.8000 28.6000) (width 0.2500) (layer "F.Cu") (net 9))
 (segment (start 15.8000 28.6000) (end 15.6000 28.4000) (width 0.2500) (layer "F.Cu") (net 9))
 (segment (start 15.6000 28.4000) (end 13.0000 28.4000) (width 0.2500) (layer "F.Cu") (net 9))
 (segment (start 24.6000 28.6000) (end 28.8000 28.6000) (width 0.2500) (layer "F.Cu") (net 7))
 (segment (start 28.8000 28.6000) (end 30.4000 27.0000) (width 0.2500) (layer "F.Cu") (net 7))
 (segment (start 30.4000 27.0000) (end 32.2000 27.0000) (width 0.2500) (layer "F.Cu") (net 7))
 (segment (start 23.0000 33.0000) (end 23.0000 31.6000) (width 0.2500) (layer "F.Cu") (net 7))
 (segment (start 23.0000 31.6000) (end 24.6000 30.0000) (width 0.2500) (layer "F.Cu") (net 7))
 (segment (start 24.6000 30.0000) (end 24.6000 28.6000) (width 0.2500) (layer "F.Cu") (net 7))
 (segment (start 24.6000 27.2000) (end 28.8000 27.2000) (width 0.2500) (layer "F.Cu") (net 12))
 (segment (start 28.8000 27.2000) (end 30.4000 25.6000) (width 0.2500) (layer "F.Cu") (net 12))
 (segment (start 30.4000 25.6000) (end 32.2000 25.6000) (width 0.2500) (layer "F.Cu") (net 12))
 (segment (start 24.6000 26.0000) (end 28.8000 26.0000) (width 0.2500) (layer "F.Cu") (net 11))
 (segment (start 28.8000 26.0000) (end 30.4000 24.4000) (width 0.2500) (layer "F.Cu") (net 11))
 (segment (start 30.4000 24.4000) (end 32.2000 24.4000) (width 0.2500) (layer "F.Cu") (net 11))
 (segment (start 24.6000 24.8000) (end 28.6000 24.8000) (width 0.2500) (layer "F.Cu") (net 10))
 (segment (start 28.6000 24.8000) (end 30.4000 23.0000) (width 0.2500) (layer "F.Cu") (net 10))
 (segment (start 30.4000 23.0000) (end 32.2000 23.0000) (width 0.2500) (layer "F.Cu") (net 10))
 (segment (start 44.0000 25.0000) (end 45.2000 26.2000) (width 0.2500) (layer "F.Cu") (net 4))
 (segment (start 45.2000 26.2000) (end 45.2000 32.2000) (width 0.2500) (layer "F.Cu") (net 4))
 (segment (start 45.2000 32.2000) (end 43.0000 34.4000) (width 0.2500) (layer "F.Cu") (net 4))
 (segment (start 36.0000 35.0000) (end 40.8000 35.0000) (width 0.2500) (layer "F.Cu") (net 4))
 (segment (start 40.8000 35.0000) (end 41.4000 34.4000) (width 0.2500) (layer "F.Cu") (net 4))
 (segment (start 41.4000 34.4000) (end 43.0000 34.4000) (width 0.2500) (layer "F.Cu") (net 4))
 (via (at 13.0000 15.8000) (size 0.6000) (drill 0.3000) (layers "F.Cu" "B.Cu") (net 2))
 (via (at 39.0000 27.0000) (size 0.6000) (drill 0.3000) (layers "F.Cu" "B.Cu") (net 2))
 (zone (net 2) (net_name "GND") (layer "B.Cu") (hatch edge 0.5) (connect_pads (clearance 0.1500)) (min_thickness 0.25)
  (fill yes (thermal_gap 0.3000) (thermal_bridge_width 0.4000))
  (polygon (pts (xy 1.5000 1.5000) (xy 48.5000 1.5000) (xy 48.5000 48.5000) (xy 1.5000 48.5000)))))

